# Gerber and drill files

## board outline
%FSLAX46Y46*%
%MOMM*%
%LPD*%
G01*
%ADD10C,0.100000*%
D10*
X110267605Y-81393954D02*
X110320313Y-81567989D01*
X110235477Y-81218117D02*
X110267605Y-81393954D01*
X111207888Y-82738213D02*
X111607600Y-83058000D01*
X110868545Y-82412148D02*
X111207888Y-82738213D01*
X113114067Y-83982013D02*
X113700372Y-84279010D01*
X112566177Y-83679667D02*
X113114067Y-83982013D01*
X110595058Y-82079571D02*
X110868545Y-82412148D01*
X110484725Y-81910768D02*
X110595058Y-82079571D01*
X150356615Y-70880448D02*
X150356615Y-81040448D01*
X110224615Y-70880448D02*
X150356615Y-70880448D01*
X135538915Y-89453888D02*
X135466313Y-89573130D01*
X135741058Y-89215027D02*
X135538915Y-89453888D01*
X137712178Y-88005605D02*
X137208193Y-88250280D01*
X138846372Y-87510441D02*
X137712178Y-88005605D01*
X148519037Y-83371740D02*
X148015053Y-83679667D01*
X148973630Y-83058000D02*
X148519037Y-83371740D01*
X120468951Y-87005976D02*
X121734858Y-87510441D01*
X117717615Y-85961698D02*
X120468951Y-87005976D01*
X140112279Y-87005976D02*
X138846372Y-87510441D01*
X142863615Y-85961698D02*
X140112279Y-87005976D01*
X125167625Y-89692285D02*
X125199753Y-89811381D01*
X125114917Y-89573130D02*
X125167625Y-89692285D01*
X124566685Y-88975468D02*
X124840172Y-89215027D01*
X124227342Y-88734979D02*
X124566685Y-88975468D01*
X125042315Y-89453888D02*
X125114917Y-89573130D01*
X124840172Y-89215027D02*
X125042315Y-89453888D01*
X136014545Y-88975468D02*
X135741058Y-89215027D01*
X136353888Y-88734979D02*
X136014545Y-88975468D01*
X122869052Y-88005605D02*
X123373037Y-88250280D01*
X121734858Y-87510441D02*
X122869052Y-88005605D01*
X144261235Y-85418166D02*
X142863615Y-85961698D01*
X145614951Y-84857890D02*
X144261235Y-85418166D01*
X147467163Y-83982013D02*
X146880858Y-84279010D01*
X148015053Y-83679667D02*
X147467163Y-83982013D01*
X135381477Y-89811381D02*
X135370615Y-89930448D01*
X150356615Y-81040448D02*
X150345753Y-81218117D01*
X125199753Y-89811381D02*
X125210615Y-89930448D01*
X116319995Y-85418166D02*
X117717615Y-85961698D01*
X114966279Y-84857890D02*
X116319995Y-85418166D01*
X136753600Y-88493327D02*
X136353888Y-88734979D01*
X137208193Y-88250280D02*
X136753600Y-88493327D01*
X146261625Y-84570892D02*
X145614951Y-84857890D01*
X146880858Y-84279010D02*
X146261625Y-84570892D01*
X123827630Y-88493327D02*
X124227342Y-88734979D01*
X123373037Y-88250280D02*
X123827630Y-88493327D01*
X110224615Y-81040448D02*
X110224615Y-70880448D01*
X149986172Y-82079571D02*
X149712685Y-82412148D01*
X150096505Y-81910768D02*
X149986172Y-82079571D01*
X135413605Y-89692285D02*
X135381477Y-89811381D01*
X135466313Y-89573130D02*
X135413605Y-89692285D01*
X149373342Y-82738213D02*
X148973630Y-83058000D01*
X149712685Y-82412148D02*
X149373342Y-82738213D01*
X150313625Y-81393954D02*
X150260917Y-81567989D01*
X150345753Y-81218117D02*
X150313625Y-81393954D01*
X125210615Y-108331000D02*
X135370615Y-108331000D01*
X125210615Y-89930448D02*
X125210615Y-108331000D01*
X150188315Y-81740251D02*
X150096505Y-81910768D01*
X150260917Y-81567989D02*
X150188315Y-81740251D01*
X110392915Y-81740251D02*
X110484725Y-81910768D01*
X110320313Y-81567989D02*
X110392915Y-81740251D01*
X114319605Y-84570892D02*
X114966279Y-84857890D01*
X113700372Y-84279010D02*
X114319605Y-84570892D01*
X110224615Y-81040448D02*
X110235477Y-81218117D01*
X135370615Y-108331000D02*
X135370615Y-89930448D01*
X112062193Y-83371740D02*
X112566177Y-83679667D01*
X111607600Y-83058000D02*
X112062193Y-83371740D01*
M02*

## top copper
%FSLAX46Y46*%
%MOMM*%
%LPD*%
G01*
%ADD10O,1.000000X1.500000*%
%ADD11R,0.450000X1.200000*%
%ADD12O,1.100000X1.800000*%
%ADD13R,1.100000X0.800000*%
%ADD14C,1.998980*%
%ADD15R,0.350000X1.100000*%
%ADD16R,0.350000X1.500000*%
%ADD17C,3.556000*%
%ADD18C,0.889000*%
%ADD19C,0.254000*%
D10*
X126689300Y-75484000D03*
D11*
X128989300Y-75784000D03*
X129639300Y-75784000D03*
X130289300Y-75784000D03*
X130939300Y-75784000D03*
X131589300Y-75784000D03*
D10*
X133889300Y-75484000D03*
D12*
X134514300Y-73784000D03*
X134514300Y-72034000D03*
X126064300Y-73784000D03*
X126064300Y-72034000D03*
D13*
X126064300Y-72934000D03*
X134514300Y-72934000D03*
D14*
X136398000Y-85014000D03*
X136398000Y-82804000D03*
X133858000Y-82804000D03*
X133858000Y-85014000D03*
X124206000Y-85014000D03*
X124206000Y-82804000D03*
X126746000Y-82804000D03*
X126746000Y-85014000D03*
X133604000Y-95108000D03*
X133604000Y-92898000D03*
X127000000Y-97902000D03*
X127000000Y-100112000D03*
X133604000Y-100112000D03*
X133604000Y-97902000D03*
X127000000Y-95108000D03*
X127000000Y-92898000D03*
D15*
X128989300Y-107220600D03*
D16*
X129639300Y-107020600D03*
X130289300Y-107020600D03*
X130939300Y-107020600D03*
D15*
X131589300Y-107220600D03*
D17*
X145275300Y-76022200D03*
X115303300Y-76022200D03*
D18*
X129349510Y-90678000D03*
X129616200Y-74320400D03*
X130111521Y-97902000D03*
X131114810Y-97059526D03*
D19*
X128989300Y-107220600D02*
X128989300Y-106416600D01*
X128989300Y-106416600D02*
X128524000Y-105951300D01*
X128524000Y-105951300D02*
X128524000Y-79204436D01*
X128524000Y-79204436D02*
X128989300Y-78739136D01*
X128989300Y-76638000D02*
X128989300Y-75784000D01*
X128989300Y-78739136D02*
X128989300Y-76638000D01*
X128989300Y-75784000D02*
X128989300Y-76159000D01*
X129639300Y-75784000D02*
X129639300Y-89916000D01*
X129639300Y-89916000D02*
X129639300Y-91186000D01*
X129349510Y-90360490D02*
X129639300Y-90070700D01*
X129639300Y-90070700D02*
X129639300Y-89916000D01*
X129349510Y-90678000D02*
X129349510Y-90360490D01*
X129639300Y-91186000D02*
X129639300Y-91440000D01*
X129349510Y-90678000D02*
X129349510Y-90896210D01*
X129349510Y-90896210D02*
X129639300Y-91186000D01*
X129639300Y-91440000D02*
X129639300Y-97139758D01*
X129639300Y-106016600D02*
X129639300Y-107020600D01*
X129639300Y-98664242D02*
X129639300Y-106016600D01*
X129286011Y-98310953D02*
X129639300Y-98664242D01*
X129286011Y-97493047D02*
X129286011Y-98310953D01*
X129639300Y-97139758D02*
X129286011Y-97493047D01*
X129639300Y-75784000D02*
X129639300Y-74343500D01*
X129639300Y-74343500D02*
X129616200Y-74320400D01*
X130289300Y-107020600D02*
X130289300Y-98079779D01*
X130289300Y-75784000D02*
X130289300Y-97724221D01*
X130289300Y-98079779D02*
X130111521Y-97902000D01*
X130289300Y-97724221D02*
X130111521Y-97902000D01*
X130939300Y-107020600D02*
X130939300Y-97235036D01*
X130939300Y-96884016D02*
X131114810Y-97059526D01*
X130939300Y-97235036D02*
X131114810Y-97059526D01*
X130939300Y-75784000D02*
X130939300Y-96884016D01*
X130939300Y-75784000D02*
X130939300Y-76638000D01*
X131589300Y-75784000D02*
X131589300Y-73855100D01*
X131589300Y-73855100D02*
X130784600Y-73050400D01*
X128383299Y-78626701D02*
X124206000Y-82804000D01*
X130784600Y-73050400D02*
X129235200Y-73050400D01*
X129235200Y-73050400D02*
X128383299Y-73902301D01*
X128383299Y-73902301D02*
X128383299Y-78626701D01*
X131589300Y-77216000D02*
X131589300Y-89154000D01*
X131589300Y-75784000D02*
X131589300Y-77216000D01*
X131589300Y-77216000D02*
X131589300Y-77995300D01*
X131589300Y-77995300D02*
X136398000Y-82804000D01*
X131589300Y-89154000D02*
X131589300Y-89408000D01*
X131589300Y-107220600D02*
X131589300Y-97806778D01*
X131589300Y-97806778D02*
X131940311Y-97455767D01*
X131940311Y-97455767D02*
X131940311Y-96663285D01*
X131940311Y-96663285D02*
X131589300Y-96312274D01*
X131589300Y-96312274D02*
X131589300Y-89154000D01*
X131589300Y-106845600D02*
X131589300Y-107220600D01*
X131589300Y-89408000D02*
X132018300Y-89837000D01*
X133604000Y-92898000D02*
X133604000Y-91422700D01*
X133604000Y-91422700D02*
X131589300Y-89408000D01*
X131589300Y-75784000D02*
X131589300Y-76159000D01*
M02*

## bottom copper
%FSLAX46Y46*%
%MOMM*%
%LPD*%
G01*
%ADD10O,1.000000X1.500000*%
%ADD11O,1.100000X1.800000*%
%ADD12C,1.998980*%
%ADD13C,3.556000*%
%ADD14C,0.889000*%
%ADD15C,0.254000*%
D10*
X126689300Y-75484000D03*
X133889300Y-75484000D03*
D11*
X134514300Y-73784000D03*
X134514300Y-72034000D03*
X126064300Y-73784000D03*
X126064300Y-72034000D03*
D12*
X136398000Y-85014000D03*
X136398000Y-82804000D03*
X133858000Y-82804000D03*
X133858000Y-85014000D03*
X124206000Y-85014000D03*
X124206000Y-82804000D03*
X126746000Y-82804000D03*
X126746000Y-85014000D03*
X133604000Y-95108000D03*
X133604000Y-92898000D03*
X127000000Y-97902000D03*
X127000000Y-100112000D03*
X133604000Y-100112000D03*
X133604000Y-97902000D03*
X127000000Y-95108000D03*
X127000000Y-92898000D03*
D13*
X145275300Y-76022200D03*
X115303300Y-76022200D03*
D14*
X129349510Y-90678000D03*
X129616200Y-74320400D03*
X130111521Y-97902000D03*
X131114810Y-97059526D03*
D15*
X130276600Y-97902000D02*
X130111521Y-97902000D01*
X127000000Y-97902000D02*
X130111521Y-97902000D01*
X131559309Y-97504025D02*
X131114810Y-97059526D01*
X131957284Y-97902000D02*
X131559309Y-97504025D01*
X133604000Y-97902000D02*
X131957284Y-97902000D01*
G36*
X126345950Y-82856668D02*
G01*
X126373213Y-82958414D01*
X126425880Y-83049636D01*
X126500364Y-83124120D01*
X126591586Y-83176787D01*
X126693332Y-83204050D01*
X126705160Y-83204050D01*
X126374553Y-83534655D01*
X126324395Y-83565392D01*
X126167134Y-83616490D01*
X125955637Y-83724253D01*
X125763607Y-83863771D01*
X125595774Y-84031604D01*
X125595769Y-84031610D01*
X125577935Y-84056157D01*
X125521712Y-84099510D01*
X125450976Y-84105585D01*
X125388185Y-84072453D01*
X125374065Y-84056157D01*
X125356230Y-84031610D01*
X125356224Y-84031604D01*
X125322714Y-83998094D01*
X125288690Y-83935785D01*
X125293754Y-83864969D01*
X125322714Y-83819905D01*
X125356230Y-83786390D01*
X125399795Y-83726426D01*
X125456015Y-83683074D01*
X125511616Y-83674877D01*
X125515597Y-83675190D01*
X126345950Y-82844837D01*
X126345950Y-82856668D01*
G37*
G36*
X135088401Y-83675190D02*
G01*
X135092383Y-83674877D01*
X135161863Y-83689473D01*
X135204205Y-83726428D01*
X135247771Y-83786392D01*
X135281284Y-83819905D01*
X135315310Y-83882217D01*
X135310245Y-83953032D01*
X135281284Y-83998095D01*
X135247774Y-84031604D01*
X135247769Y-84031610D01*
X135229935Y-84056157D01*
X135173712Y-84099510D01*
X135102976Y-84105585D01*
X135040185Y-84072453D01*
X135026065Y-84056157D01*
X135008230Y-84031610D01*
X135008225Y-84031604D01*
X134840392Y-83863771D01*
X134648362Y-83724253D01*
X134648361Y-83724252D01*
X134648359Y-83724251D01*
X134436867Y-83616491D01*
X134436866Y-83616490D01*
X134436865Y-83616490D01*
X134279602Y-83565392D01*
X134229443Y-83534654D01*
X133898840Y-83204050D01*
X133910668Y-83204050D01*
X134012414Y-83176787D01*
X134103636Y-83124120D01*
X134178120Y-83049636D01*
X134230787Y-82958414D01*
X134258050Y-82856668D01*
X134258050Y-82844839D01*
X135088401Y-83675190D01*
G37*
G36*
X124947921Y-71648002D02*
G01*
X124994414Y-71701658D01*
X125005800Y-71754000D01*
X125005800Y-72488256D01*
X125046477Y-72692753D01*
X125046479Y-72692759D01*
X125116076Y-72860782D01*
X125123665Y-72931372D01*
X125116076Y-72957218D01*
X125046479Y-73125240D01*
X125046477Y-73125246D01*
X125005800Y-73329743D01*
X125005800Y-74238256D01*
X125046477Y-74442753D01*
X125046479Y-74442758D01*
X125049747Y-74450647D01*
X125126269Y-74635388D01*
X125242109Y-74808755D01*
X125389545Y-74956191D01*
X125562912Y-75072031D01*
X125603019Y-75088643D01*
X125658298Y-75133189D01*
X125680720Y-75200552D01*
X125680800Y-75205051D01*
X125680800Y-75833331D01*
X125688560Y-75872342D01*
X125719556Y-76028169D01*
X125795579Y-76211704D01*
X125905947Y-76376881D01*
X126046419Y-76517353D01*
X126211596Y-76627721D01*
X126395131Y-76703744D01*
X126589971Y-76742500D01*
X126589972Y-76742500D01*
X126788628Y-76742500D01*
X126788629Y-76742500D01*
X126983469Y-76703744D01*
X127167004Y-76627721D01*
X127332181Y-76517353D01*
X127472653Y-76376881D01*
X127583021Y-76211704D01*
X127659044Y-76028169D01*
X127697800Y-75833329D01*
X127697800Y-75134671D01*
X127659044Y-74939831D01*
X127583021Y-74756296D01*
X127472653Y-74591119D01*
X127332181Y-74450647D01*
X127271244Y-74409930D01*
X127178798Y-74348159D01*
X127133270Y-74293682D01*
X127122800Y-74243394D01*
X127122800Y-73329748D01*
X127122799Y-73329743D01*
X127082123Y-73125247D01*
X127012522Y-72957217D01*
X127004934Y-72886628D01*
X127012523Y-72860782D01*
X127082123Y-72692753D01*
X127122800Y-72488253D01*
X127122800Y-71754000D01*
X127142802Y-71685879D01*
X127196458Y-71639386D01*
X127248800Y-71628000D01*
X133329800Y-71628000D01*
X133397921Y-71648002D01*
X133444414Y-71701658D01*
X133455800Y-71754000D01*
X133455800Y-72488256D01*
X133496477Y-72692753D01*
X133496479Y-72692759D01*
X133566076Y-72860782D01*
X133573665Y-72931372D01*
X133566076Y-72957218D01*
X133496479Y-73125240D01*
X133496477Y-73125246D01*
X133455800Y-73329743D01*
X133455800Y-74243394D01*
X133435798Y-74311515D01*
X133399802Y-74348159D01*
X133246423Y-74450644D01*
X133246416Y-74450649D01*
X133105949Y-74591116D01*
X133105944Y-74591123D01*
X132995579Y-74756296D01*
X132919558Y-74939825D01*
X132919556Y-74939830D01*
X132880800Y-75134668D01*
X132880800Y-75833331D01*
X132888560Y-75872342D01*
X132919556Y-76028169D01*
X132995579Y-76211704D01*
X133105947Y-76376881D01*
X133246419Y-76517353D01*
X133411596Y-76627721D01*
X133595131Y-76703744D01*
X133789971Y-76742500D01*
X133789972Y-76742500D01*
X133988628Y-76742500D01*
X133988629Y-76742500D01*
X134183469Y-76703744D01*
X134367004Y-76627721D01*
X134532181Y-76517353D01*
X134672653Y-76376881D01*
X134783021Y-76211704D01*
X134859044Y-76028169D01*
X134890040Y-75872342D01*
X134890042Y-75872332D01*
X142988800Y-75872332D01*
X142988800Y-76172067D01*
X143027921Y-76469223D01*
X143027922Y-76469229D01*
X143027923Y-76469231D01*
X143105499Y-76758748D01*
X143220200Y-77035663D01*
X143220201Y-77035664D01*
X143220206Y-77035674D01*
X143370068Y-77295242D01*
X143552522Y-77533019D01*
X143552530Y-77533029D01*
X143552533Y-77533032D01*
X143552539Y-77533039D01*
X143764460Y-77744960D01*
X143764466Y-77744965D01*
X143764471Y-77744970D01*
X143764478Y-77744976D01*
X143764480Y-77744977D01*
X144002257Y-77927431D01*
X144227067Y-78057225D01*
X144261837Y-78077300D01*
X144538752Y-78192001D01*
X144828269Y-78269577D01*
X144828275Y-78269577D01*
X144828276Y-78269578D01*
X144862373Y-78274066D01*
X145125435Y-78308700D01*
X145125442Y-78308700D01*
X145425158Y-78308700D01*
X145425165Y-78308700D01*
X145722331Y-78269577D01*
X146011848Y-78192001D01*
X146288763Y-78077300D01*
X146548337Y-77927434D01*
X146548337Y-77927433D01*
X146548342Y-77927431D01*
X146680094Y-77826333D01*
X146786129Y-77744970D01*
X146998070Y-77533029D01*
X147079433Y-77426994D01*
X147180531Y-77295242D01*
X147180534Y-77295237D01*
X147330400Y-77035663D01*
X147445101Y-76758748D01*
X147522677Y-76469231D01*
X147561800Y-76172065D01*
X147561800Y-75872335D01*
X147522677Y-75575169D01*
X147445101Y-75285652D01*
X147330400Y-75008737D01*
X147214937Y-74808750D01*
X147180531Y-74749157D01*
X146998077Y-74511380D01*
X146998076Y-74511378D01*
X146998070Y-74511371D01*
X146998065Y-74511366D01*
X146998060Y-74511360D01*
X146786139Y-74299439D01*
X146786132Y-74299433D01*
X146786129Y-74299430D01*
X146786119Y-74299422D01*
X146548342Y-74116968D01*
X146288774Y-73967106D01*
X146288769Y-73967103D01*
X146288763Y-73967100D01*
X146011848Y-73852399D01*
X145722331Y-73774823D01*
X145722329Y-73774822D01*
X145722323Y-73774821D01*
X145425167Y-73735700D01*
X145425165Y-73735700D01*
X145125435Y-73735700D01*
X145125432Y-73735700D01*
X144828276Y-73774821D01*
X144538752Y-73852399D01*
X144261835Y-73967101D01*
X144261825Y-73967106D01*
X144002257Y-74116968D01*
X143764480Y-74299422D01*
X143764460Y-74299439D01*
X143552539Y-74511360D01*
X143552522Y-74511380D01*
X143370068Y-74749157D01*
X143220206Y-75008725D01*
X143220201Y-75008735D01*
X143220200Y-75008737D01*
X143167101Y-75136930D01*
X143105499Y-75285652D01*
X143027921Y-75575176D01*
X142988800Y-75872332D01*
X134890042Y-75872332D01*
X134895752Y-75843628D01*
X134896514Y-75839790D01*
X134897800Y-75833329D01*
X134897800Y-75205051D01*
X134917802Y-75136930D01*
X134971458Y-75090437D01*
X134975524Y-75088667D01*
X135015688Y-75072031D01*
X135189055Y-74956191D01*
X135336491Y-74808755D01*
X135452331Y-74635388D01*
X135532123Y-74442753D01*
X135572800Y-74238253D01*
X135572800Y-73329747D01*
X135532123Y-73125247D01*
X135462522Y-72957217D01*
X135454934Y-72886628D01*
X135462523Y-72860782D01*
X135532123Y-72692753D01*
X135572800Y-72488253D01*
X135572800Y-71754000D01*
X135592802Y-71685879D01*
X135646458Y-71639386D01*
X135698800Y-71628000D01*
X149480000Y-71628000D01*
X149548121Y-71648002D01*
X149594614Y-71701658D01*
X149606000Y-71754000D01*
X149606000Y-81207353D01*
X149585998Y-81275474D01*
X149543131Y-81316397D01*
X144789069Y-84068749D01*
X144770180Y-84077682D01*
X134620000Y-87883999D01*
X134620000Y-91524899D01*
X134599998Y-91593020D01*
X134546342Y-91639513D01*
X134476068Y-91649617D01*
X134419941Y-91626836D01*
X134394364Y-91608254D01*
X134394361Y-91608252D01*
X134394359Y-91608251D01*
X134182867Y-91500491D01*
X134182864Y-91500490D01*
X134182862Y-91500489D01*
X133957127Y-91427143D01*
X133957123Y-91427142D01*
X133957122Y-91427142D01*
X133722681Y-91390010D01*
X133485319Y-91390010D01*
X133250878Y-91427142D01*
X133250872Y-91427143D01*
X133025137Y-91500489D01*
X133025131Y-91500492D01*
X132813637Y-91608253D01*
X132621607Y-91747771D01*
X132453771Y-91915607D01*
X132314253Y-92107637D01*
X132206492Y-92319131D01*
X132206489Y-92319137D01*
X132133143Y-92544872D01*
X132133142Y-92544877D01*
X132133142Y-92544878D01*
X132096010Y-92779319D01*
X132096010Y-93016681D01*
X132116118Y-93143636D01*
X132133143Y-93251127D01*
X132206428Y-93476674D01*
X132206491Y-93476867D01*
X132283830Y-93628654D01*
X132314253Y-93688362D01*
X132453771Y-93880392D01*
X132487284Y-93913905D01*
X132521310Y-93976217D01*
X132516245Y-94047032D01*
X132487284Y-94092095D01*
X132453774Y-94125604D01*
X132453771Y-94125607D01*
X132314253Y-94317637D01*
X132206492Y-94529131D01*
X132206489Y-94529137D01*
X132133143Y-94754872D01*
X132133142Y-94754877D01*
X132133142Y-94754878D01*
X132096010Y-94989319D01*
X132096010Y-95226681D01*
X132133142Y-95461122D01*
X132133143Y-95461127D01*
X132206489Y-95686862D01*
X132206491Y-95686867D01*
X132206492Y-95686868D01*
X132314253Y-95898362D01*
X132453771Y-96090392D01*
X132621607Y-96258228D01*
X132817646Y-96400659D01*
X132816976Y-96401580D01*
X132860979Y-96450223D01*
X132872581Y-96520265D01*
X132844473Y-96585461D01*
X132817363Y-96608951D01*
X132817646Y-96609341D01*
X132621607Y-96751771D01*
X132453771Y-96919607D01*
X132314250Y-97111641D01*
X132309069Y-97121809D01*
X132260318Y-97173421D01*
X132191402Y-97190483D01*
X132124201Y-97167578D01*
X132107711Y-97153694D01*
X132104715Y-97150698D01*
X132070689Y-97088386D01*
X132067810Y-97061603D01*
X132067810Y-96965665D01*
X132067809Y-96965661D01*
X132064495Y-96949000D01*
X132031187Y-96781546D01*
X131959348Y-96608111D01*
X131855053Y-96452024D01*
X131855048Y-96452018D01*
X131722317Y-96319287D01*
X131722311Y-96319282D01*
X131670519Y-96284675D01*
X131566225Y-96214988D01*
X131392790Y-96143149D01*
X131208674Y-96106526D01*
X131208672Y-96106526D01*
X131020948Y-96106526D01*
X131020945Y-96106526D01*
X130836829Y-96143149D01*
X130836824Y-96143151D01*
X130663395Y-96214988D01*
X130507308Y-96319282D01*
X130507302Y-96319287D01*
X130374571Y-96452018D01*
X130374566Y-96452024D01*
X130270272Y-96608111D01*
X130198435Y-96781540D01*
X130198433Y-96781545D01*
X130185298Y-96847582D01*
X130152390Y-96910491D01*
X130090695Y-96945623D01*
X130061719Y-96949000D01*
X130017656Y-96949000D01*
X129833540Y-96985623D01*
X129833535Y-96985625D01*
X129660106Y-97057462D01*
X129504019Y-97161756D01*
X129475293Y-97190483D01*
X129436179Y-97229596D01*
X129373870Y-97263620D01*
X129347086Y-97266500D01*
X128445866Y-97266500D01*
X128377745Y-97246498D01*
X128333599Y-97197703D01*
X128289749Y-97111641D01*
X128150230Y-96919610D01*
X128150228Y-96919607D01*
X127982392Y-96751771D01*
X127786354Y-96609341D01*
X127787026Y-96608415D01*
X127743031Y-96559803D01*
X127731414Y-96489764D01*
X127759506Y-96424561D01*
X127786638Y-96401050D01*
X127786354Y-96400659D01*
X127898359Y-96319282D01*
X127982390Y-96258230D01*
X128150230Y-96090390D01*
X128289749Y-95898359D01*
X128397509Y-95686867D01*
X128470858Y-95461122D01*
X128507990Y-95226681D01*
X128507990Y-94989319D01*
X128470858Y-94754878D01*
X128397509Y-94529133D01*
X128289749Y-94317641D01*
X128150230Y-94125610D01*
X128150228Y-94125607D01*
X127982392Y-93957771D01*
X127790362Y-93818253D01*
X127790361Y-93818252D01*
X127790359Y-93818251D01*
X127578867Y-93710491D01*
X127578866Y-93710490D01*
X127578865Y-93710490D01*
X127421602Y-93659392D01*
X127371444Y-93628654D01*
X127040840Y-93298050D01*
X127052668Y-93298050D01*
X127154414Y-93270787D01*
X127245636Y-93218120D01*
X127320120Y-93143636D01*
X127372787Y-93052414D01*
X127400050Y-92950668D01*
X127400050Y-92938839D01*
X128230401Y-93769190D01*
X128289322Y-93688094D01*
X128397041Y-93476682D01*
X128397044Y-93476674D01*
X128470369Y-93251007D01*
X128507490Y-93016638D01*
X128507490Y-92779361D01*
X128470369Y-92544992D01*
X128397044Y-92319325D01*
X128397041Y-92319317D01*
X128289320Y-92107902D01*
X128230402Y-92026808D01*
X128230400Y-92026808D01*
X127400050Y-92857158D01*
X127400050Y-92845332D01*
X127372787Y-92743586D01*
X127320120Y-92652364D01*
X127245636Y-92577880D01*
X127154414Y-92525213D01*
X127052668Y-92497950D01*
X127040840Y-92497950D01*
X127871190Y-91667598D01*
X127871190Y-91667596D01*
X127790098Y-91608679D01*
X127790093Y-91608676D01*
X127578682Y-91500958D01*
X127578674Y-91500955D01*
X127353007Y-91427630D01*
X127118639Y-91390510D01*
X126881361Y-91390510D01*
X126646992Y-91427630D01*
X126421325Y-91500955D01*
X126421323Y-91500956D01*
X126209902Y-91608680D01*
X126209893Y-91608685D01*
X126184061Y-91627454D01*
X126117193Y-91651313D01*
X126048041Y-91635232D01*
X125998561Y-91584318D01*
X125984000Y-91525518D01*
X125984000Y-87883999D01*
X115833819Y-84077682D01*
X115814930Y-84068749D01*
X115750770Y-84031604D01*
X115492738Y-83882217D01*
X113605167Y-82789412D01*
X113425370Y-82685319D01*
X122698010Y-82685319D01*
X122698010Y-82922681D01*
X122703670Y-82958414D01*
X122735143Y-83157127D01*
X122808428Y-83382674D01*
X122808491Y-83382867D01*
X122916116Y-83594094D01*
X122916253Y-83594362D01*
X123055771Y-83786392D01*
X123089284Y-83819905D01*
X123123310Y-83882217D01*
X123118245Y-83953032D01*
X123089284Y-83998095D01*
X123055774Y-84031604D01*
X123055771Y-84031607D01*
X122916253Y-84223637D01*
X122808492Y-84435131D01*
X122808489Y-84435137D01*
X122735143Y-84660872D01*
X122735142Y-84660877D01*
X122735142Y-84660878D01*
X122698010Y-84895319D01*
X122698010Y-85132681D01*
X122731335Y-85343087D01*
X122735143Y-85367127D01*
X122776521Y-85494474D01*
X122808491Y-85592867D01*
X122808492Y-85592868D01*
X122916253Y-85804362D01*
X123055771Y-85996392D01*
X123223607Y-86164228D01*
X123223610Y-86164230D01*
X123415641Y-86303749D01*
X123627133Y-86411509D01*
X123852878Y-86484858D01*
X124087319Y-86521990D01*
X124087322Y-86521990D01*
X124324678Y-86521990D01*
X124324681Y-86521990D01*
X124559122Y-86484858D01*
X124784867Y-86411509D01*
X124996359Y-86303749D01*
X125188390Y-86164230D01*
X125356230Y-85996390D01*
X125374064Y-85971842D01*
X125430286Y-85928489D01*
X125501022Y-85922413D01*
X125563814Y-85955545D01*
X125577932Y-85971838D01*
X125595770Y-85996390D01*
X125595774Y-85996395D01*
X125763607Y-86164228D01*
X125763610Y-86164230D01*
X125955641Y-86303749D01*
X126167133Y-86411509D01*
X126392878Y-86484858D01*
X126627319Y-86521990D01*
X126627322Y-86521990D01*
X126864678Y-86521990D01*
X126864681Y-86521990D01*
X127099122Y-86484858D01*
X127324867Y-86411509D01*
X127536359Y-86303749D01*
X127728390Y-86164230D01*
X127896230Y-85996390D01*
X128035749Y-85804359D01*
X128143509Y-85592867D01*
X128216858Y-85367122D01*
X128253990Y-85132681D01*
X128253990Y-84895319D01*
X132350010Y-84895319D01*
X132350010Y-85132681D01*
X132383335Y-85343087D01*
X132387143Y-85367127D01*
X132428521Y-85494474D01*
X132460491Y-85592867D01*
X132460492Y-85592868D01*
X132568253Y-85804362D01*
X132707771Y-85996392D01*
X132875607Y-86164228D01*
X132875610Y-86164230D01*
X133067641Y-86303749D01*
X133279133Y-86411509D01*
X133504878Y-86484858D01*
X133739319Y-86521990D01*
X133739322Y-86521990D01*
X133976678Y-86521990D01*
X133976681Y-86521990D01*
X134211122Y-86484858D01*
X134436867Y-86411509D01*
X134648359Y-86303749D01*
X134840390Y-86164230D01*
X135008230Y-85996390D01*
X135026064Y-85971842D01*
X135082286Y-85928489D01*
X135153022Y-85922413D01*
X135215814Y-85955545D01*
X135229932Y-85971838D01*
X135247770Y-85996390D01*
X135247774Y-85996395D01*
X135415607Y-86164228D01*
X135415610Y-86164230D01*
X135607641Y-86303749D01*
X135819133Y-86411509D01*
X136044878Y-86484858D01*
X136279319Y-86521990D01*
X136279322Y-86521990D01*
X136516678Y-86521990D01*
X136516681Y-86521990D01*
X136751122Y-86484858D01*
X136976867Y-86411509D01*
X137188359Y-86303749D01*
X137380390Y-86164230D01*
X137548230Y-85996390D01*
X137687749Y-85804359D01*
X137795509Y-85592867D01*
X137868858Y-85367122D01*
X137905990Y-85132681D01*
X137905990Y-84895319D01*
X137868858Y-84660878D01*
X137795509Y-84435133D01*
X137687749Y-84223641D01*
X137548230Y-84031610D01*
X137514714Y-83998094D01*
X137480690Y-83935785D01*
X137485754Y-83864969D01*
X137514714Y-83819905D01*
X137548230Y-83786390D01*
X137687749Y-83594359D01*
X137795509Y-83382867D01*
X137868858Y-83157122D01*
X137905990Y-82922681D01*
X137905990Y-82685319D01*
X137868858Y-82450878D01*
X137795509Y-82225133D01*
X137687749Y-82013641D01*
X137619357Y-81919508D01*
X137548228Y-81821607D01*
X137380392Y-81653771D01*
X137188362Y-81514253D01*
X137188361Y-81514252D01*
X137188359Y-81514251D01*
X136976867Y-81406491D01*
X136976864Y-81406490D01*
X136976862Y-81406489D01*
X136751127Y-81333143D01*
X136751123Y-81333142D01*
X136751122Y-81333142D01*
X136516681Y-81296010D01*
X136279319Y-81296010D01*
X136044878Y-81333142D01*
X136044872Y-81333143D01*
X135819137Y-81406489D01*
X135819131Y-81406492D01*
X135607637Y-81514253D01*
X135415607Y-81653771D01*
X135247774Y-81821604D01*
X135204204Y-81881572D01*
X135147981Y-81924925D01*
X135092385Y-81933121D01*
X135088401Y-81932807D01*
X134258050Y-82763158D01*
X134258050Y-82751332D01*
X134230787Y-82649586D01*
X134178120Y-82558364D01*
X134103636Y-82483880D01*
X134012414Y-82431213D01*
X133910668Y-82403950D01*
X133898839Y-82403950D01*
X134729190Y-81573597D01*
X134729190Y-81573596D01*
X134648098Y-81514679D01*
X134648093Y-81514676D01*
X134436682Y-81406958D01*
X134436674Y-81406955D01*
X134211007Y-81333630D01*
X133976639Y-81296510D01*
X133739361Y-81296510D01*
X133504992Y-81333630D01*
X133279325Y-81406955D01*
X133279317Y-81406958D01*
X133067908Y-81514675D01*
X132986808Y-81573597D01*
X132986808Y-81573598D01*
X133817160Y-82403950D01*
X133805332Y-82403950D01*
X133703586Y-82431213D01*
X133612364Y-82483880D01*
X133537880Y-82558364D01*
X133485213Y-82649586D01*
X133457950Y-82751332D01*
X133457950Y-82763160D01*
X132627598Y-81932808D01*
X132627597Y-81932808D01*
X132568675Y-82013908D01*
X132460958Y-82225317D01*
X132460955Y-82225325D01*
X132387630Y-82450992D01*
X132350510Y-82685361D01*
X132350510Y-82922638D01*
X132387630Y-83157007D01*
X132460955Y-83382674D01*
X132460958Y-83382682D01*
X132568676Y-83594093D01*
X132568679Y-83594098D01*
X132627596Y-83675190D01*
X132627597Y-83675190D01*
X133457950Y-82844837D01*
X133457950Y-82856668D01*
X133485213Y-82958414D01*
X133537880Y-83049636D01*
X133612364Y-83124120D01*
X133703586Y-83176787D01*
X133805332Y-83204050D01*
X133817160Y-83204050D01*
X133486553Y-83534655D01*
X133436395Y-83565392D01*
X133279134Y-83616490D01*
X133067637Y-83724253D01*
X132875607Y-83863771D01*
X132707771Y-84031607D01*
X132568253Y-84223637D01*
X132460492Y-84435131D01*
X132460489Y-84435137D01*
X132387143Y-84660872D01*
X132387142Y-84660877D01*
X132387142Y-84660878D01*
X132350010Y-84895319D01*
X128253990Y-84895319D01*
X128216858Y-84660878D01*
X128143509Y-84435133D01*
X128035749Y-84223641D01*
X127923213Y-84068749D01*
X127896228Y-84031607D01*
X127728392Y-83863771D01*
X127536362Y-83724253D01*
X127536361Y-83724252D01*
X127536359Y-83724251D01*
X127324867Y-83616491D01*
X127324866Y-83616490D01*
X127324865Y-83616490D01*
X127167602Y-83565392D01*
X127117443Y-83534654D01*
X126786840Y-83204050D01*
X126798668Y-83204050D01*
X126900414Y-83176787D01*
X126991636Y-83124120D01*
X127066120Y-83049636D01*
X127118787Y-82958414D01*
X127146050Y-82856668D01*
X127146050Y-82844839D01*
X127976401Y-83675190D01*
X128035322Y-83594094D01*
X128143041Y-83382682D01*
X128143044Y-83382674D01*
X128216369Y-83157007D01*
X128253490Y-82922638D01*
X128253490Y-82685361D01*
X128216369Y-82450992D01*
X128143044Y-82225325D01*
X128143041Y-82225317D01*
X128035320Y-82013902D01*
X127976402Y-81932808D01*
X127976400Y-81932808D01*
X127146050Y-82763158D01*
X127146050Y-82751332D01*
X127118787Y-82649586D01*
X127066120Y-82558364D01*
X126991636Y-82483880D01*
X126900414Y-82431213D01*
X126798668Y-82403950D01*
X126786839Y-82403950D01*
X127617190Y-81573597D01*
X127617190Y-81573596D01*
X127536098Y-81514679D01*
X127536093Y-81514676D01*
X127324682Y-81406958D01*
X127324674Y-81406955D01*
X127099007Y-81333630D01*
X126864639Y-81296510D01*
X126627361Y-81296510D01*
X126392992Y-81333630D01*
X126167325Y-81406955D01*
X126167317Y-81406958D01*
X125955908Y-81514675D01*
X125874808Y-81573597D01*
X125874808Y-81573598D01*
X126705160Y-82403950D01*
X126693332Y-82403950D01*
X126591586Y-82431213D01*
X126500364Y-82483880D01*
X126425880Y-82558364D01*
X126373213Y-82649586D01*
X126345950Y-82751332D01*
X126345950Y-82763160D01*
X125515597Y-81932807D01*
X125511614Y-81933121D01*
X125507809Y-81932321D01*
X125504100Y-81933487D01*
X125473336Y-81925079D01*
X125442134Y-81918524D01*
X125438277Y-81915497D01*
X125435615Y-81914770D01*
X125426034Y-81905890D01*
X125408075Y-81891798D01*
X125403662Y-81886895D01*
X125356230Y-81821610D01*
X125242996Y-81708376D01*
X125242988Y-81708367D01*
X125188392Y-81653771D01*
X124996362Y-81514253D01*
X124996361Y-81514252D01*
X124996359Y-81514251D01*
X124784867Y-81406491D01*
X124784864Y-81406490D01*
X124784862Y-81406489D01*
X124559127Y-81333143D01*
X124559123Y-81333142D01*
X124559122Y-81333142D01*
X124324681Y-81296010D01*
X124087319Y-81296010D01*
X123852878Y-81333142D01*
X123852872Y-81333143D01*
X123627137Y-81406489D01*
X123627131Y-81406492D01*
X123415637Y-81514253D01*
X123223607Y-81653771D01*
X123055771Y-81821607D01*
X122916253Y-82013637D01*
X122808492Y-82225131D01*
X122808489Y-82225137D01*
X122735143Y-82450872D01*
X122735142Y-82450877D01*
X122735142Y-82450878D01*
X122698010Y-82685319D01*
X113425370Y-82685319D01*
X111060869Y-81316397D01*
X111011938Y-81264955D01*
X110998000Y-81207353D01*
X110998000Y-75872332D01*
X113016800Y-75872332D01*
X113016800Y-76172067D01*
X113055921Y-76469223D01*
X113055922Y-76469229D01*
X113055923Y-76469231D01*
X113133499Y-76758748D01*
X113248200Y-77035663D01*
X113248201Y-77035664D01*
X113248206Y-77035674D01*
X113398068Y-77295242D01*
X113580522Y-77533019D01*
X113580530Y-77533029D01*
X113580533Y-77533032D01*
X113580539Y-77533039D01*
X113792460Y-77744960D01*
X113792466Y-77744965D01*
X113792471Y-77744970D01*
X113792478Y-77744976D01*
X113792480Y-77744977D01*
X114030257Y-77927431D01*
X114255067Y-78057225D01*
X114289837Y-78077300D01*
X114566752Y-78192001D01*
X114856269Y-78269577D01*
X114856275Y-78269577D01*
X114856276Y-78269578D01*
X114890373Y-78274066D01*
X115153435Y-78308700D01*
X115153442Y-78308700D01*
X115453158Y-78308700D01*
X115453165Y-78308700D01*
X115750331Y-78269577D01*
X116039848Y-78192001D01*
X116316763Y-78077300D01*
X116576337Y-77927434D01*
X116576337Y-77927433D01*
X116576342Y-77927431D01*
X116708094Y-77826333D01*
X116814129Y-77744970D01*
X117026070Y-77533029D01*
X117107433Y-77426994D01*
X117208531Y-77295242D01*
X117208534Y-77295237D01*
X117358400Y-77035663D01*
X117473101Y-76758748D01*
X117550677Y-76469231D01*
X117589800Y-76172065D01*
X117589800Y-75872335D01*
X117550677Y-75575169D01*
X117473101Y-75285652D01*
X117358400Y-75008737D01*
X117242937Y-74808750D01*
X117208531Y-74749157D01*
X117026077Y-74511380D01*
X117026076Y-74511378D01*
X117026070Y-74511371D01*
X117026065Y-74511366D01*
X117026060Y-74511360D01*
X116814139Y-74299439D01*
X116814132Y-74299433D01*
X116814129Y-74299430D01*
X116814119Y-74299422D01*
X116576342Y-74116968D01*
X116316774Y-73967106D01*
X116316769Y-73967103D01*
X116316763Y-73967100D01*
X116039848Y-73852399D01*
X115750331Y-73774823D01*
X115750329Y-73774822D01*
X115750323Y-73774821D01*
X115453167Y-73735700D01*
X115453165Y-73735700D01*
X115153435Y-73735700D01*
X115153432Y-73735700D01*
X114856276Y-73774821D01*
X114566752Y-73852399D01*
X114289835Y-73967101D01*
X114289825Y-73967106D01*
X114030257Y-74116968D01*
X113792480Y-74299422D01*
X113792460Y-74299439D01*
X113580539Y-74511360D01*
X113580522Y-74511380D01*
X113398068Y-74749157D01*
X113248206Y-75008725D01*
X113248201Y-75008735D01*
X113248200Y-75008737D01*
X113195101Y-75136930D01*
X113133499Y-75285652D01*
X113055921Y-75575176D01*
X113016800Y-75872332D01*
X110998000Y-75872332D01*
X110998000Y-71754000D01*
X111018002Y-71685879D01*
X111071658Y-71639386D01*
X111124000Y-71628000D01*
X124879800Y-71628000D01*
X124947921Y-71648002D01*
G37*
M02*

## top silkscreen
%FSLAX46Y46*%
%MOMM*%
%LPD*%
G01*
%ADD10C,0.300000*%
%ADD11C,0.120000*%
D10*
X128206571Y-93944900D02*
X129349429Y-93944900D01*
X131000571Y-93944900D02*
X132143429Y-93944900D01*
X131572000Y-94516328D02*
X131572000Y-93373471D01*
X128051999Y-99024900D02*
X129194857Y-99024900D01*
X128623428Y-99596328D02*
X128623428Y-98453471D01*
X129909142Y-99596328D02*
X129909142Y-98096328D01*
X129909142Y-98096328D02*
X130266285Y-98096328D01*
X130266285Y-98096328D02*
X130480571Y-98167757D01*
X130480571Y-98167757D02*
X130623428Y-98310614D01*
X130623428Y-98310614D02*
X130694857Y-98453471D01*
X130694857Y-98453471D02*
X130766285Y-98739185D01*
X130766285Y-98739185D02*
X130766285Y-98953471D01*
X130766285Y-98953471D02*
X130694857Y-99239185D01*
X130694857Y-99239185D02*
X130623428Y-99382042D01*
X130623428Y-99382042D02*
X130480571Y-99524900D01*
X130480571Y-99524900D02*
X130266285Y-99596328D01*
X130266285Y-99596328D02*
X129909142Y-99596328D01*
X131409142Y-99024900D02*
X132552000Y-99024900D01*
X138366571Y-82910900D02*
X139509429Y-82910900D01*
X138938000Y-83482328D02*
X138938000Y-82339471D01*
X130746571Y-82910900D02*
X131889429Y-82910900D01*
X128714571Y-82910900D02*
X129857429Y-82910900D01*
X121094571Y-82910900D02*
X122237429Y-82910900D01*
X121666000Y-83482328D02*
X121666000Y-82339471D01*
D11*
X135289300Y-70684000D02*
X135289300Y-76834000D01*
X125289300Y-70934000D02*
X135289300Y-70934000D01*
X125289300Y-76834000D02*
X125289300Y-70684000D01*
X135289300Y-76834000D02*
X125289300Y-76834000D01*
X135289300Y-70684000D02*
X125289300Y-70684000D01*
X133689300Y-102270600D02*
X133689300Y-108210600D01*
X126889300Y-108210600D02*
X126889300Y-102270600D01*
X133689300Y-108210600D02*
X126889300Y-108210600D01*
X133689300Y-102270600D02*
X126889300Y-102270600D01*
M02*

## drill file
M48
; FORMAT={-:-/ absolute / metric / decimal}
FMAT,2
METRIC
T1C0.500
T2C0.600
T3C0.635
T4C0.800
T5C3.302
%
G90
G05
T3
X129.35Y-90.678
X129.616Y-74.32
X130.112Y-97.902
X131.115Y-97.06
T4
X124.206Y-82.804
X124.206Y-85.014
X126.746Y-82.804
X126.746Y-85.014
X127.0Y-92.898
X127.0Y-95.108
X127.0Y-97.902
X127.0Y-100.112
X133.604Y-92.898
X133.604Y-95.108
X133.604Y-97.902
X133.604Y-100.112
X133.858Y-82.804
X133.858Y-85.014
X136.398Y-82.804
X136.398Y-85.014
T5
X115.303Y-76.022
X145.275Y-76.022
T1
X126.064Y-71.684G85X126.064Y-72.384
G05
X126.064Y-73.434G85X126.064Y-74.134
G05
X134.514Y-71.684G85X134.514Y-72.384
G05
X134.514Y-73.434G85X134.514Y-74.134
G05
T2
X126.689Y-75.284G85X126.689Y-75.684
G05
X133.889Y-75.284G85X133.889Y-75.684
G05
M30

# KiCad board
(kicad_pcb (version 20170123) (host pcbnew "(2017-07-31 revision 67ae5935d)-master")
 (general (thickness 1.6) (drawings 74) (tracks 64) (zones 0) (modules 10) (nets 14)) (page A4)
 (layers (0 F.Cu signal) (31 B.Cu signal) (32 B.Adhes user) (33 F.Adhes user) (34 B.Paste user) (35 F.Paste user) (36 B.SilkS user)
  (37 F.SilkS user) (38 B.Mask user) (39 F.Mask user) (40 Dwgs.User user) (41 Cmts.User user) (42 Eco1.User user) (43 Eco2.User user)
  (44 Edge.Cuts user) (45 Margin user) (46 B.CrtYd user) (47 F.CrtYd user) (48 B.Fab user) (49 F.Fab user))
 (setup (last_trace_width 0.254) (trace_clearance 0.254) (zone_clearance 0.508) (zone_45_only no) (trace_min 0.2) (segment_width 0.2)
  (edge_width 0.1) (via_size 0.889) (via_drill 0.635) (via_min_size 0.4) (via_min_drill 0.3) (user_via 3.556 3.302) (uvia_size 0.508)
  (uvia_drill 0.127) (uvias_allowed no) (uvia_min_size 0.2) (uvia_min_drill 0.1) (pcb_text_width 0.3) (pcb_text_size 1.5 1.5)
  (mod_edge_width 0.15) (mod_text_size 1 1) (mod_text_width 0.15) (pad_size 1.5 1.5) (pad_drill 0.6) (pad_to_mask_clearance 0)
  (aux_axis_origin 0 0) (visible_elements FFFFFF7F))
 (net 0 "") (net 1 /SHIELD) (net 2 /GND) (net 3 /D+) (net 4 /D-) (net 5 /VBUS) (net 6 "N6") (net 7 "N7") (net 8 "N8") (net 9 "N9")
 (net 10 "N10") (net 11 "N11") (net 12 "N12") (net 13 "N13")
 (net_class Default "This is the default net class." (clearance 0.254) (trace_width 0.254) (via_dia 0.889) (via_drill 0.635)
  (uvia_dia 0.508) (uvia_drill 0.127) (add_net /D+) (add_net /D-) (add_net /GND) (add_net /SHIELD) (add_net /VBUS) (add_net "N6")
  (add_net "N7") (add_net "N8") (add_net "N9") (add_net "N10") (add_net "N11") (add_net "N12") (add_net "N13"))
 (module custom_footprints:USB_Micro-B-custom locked (layer F.Cu) (at 130.2893 75.184 180)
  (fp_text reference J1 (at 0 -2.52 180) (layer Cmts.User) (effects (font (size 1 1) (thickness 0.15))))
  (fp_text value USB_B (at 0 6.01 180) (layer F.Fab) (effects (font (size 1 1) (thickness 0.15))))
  (fp_line (start -5 4.5) (end -5 -1.65) (layer F.SilkS) (width 0.12))
  (fp_line (start 5 4.25) (end -5 4.25) (layer F.SilkS) (width 0.12))
  (fp_line (start 5 -1.65) (end 5 4.5) (layer F.SilkS) (width 0.12))
  (fp_line (start -5 -1.65) (end 5 -1.65) (layer F.SilkS) (width 0.12))
  (fp_line (start -5 4.5) (end 5 4.5) (layer F.SilkS) (width 0.12))
  (pad "" thru_hole oval (at 3.6 -0.3 270) (size 1.5 1) (drill oval 1 0.6) (layers *.Cu *.Mask))
  (pad 5 smd rect (at 1.3 -0.6 270) (size 1.2 0.45) (layers F.Cu F.Paste F.Mask) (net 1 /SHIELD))
  (pad 4 smd rect (at 0.65 -0.6 270) (size 1.2 0.45) (layers F.Cu F.Paste F.Mask) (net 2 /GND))
  (pad 3 smd rect (at 0 -0.6 270) (size 1.2 0.45) (layers F.Cu F.Paste F.Mask) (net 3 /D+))
  (pad 2 smd rect (at -0.65 -0.6 270) (size 1.2 0.45) (layers F.Cu F.Paste F.Mask) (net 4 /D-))
  (pad 1 smd rect (at -1.3 -0.6 270) (size 1.2 0.45) (layers F.Cu F.Paste F.Mask) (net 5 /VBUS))
  (pad "" thru_hole oval (at -3.6 -0.3 270) (size 1.5 1) (drill oval 1 0.6) (layers *.Cu *.Mask))
  (pad "" thru_hole oval (at -4.225 1.4 270) (size 1.8 1.1) (drill oval 1.2 0.5) (layers *.Cu *.Mask))
  (pad "" thru_hole oval (at -4.225 3.15 270) (size 1.8 1.1) (drill oval 1.2 0.5) (layers *.Cu *.Mask))
  (pad "" thru_hole oval (at 4.225 1.4 270) (size 1.8 1.1) (drill oval 1.2 0.5) (layers *.Cu *.Mask))
  (pad "" thru_hole oval (at 4.225 3.15 270) (size 1.8 1.1) (drill oval 1.2 0.5) (layers *.Cu *.Mask))
  (pad "" smd rect (at 4.225 2.25 270) (size 0.8 1.1) (layers F.Cu F.Paste F.Mask))
  (pad "" smd rect (at -4.225 2.25 270) (size 0.8 1.1) (layers F.Cu F.Paste F.Mask)))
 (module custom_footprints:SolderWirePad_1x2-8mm (layer F.Cu) (at 136.398 83.914 270)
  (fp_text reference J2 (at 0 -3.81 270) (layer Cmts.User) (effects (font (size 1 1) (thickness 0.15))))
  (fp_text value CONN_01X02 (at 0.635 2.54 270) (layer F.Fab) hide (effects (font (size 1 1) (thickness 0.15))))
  (pad 2 thru_hole circle (at 1.1 0 270) (size 1.99898 1.99898) (drill 0.8001) (layers *.Cu *.Mask) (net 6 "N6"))
  (pad 1 thru_hole circle (at -1.11 0 270) (size 1.99898 1.99898) (drill 0.8001) (layers *.Cu *.Mask) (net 5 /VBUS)))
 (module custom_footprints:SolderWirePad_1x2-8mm (layer F.Cu) (at 133.858 83.914 270)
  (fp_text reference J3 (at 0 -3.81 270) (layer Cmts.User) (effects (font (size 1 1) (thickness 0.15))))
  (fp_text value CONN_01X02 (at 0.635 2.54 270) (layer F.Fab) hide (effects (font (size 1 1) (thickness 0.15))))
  (pad 1 thru_hole circle (at -1.11 0 270) (size 1.99898 1.99898) (drill 0.8001) (layers *.Cu *.Mask) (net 2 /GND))
  (pad 2 thru_hole circle (at 1.1 0 270) (size 1.99898 1.99898) (drill 0.8001) (layers *.Cu *.Mask) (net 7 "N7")))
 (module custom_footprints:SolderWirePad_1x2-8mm (layer F.Cu) (at 124.206 83.914 270)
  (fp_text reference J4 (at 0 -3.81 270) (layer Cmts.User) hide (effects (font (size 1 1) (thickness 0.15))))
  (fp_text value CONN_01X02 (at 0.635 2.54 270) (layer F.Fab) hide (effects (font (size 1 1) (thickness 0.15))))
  (pad 2 thru_hole circle (at 1.1 0 270) (size 1.99898 1.99898) (drill 0.8001) (layers *.Cu *.Mask) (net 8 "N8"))
  (pad 1 thru_hole circle (at -1.11 0 270) (size 1.99898 1.99898) (drill 0.8001) (layers *.Cu *.Mask) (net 5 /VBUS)))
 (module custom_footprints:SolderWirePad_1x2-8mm (layer F.Cu) (at 126.746 83.914 270)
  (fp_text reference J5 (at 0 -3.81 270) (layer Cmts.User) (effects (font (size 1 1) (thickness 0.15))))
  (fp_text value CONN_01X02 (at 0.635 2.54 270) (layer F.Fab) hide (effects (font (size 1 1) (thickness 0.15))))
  (pad 1 thru_hole circle (at -1.11 0 270) (size 1.99898 1.99898) (drill 0.8001) (layers *.Cu *.Mask) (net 2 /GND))
  (pad 2 thru_hole circle (at 1.1 0 270) (size 1.99898 1.99898) (drill 0.8001) (layers *.Cu *.Mask) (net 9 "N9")))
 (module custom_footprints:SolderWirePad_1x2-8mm (layer F.Cu) (at 133.604 94.008 270)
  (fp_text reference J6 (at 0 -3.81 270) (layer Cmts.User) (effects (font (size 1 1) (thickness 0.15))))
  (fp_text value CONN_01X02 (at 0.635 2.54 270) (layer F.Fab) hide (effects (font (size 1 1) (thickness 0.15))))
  (pad 2 thru_hole circle (at 1.1 0 270) (size 1.99898 1.99898) (drill 0.8001) (layers *.Cu *.Mask) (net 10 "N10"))
  (pad 1 thru_hole circle (at -1.11 0 270) (size 1.99898 1.99898) (drill 0.8001) (layers *.Cu *.Mask) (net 5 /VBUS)))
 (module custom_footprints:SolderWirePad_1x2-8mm (layer F.Cu) (at 127 99.012 270)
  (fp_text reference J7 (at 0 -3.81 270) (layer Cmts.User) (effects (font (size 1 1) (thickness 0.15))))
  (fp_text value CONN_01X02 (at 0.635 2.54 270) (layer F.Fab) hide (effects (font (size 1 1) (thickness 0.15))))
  (pad 1 thru_hole circle (at -1.11 0 270) (size 1.99898 1.99898) (drill 0.8001) (layers *.Cu *.Mask) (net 3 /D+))
  (pad 2 thru_hole circle (at 1.1 0 270) (size 1.99898 1.99898) (drill 0.8001) (layers *.Cu *.Mask) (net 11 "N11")))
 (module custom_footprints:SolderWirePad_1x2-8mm (layer F.Cu) (at 133.604 99.012 270)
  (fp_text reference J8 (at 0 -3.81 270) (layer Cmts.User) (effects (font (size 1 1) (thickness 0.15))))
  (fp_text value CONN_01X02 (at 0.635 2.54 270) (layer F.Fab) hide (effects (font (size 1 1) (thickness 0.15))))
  (pad 2 thru_hole circle (at 1.1 0 270) (size 1.99898 1.99898) (drill 0.8001) (layers *.Cu *.Mask) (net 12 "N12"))
  (pad 1 thru_hole circle (at -1.11 0 270) (size 1.99898 1.99898) (drill 0.8001) (layers *.Cu *.Mask) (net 4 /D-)))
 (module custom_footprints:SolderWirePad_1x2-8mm (layer F.Cu) (at 127 94.008 270)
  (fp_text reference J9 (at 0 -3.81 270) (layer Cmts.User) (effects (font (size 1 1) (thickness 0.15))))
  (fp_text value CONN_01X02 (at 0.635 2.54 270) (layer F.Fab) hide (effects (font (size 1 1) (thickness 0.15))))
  (pad 2 thru_hole circle (at 1.1 0 270) (size 1.99898 1.99898) (drill 0.8001) (layers *.Cu *.Mask) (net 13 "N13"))
  (pad 1 thru_hole circle (at -1.11 0 270) (size 1.99898 1.99898) (drill 0.8001) (layers *.Cu *.Mask) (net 2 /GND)))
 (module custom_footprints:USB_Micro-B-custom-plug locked (layer F.Cu) (at 130.2893 107.0206 180)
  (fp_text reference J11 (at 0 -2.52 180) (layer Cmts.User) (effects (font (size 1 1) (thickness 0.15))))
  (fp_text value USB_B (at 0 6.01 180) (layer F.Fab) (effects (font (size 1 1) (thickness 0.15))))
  (fp_line (start -3.4 4.75) (end -3.4 -1.19) (layer F.SilkS) (width 0.12))
  (fp_line (start 3.4 -1.19) (end 3.4 4.75) (layer F.SilkS) (width 0.12))
  (fp_line (start -3.4 -1.19) (end 3.4 -1.19) (layer F.SilkS) (width 0.12))
  (fp_line (start -3.4 4.75) (end 3.4 4.75) (layer F.SilkS) (width 0.12))
  (pad 5 smd rect (at 1.3 -0.2 270) (size 1.1 0.35) (layers F.Cu F.Paste F.Mask) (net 1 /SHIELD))
  (pad 4 smd rect (at 0.65 0 270) (size 1.5 0.35) (layers F.Cu F.Paste F.Mask) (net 2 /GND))
  (pad 3 smd rect (at 0 0 270) (size 1.5 0.35) (layers F.Cu F.Paste F.Mask) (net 3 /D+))
  (pad 2 smd rect (at -0.65 0 270) (size 1.5 0.35) (layers F.Cu F.Paste F.Mask) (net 4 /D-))
  (pad 1 smd rect (at -1.3 -0.2 270) (size 1.1 0.35) (layers F.Cu F.Paste F.Mask) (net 5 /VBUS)))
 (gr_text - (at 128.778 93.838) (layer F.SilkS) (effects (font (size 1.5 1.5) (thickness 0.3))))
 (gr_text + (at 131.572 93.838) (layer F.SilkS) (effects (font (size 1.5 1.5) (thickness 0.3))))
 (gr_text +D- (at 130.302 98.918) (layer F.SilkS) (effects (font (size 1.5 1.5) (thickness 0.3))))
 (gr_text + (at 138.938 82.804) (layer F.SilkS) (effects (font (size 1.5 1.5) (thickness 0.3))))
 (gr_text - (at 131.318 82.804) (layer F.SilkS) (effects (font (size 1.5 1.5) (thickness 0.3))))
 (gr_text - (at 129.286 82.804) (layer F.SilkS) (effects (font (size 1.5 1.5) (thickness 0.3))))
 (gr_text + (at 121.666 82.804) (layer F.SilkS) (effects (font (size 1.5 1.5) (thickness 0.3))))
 (gr_line (start 110.267605 81.393954) (end 110.320313 81.567989) (layer Edge.Cuts) (width 0.1))
 (gr_line (start 110.235477 81.218117) (end 110.267605 81.393954) (layer Edge.Cuts) (width 0.1))
 (gr_line (start 111.207888 82.738213) (end 111.6076 83.058) (layer Edge.Cuts) (width 0.1))
 (gr_line (start 110.868545 82.412148) (end 111.207888 82.738213) (layer Edge.Cuts) (width 0.1))
 (gr_line (start 113.114067 83.982013) (end 113.700372 84.27901) (layer Edge.Cuts) (width 0.1))
 (gr_line (start 112.566177 83.679667) (end 113.114067 83.982013) (layer Edge.Cuts) (width 0.1))
 (gr_line (start 110.595058 82.079571) (end 110.868545 82.412148) (layer Edge.Cuts) (width 0.1))
 (gr_line (start 110.484725 81.910768) (end 110.595058 82.079571) (layer Edge.Cuts) (width 0.1))
 (gr_line (start 150.356615 70.880448) (end 150.356615 81.040448) (layer Edge.Cuts) (width 0.1))
 (gr_line (start 110.224615 70.880448) (end 150.356615 70.880448) (layer Edge.Cuts) (width 0.1))
 (gr_line (start 135.538915 89.453888) (end 135.466313 89.57313) (layer Edge.Cuts) (width 0.1))
 (gr_line (start 135.741058 89.215027) (end 135.538915 89.453888) (layer Edge.Cuts) (width 0.1))
 (gr_line (start 137.712178 88.005605) (end 137.208193 88.25028) (layer Edge.Cuts) (width 0.1))
 (gr_line (start 138.846372 87.510441) (end 137.712178 88.005605) (layer Edge.Cuts) (width 0.1))
 (gr_line (start 148.519037 83.37174) (end 148.015053 83.679667) (layer Edge.Cuts) (width 0.1))
 (gr_line (start 148.97363 83.058) (end 148.519037 83.37174) (layer Edge.Cuts) (width 0.1))
 (gr_line (start 120.468951 87.005976) (end 121.734858 87.510441) (layer Edge.Cuts) (width 0.1))
 (gr_line (start 117.717615 85.961698) (end 120.468951 87.005976) (layer Edge.Cuts) (width 0.1))
 (gr_line (start 140.112279 87.005976) (end 138.846372 87.510441) (layer Edge.Cuts) (width 0.1))
 (gr_line (start 142.863615 85.961698) (end 140.112279 87.005976) (layer Edge.Cuts) (width 0.1))
 (gr_line (start 125.167625 89.692285) (end 125.199753 89.811381) (layer Edge.Cuts) (width 0.1))
 (gr_line (start 125.114917 89.57313) (end 125.167625 89.692285) (layer Edge.Cuts) (width 0.1))
 (gr_line (start 124.566685 88.975468) (end 124.840172 89.215027) (layer Edge.Cuts) (width 0.1))
 (gr_line (start 124.227342 88.734979) (end 124.566685 88.975468) (layer Edge.Cuts) (width 0.1))
 (gr_line (start 125.042315 89.453888) (end 125.114917 89.57313) (layer Edge.Cuts) (width 0.1))
 (gr_line (start 124.840172 89.215027) (end 125.042315 89.453888) (layer Edge.Cuts) (width 0.1))
 (gr_line (start 136.014545 88.975468) (end 135.741058 89.215027) (layer Edge.Cuts) (width 0.1))
 (gr_line (start 136.353888 88.734979) (end 136.014545 88.975468) (layer Edge.Cuts) (width 0.1))
 (gr_line (start 122.869052 88.005605) (end 123.373037 88.25028) (layer Edge.Cuts) (width 0.1))
 (gr_line (start 121.734858 87.510441) (end 122.869052 88.005605) (layer Edge.Cuts) (width 0.1))
 (gr_line (start 144.261235 85.418166) (end 142.863615 85.961698) (layer Edge.Cuts) (width 0.1))
 (gr_line (start 145.614951 84.85789) (end 144.261235 85.418166) (layer Edge.Cuts) (width 0.1))
 (gr_line (start 147.467163 83.982013) (end 146.880858 84.27901) (layer Edge.Cuts) (width 0.1))
 (gr_line (start 148.015053 83.679667) (end 147.467163 83.982013) (layer Edge.Cuts) (width 0.1))
 (gr_line (start 135.381477 89.811381) (end 135.370615 89.930448) (layer Edge.Cuts) (width 0.1))
 (gr_line (start 150.356615 81.040448) (end 150.345753 81.218117) (layer Edge.Cuts) (width 0.1))
 (gr_line (start 125.199753 89.811381) (end 125.210615 89.930448) (layer Edge.Cuts) (width 0.1))
 (gr_line (start 116.319995 85.418166) (end 117.717615 85.961698) (layer Edge.Cuts) (width 0.1))
 (gr_line (start 114.966279 84.85789) (end 116.319995 85.418166) (layer Edge.Cuts) (width 0.1))
 (gr_line (start 136.7536 88.493327) (end 136.353888 88.734979) (layer Edge.Cuts) (width 0.1))
 (gr_line (start 137.208193 88.25028) (end 136.7536 88.493327) (layer Edge.Cuts) (width 0.1))
 (gr_line (start 146.261625 84.570892) (end 145.614951 84.85789) (layer Edge.Cuts) (width 0.1))
 (gr_line (start 146.880858 84.27901) (end 146.261625 84.570892) (layer Edge.Cuts) (width 0.1))
 (gr_line (start 123.82763 88.493327) (end 124.227342 88.734979) (layer Edge.Cuts) (width 0.1))
 (gr_line (start 123.373037 88.25028) (end 123.82763 88.493327) (layer Edge.Cuts) (width 0.1))
 (gr_line (start 110.224615 81.040448) (end 110.224615 70.880448) (layer Edge.Cuts) (width 0.1))
 (gr_line (start 149.986172 82.079571) (end 149.712685 82.412148) (layer Edge.Cuts) (width 0.1))
 (gr_line (start 150.096505 81.910768) (end 149.986172 82.079571) (layer Edge.Cuts) (width 0.1))
 (gr_line (start 135.413605 89.692285) (end 135.381477 89.811381) (layer Edge.Cuts) (width 0.1))
 (gr_line (start 135.466313 89.57313) (end 135.413605 89.692285) (layer Edge.Cuts) (width 0.1))
 (gr_line (start 149.373342 82.738213) (end 148.97363 83.058) (layer Edge.Cuts) (width 0.1))
 (gr_line (start 149.712685 82.412148) (end 149.373342 82.738213) (layer Edge.Cuts) (width 0.1))
 (gr_line (start 150.313625 81.393954) (end 150.260917 81.567989) (layer Edge.Cuts) (width 0.1))
 (gr_line (start 150.345753 81.218117) (end 150.313625 81.393954) (layer Edge.Cuts) (width 0.1))
 (gr_line (start 125.210615 108.331) (end 135.370615 108.331) (layer Edge.Cuts) (width 0.1))
 (gr_line (start 125.210615 89.930448) (end 125.210615 108.331) (layer Edge.Cuts) (width 0.1))
 (gr_line (start 150.188315 81.740251) (end 150.096505 81.910768) (layer Edge.Cuts) (width 0.1))
 (gr_line (start 150.260917 81.567989) (end 150.188315 81.740251) (layer Edge.Cuts) (width 0.1))
 (gr_line (start 110.392915 81.740251) (end 110.484725 81.910768) (layer Edge.Cuts) (width 0.1))
 (gr_line (start 110.320313 81.567989) (end 110.392915 81.740251) (layer Edge.Cuts) (width 0.1))
 (gr_line (start 114.319605 84.570892) (end 114.966279 84.85789) (layer Edge.Cuts) (width 0.1))
 (gr_line (start 113.700372 84.27901) (end 114.319605 84.570892) (layer Edge.Cuts) (width 0.1))
 (gr_line (start 110.224615 81.040448) (end 110.235477 81.218117) (layer Edge.Cuts) (width 0.1))
 (gr_line (start 135.370615 108.331) (end 135.370615 89.930448) (layer Edge.Cuts) (width 0.1))
 (gr_line (start 112.062193 83.37174) (end 112.566177 83.679667) (layer Edge.Cuts) (width 0.1))
 (gr_line (start 111.6076 83.058) (end 112.062193 83.37174) (layer Edge.Cuts) (width 0.1))
 (via (at 145.2753 76.0222) (size 3.556) (drill 3.302) (layers F.Cu B.Cu) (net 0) (status 40000))
 (via (at 115.3033 76.0222) (size 3.556) (drill 3.302) (layers F.Cu B.Cu) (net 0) (status 40000))
 (segment (start 128.9893 107.2206) (end 128.9893 106.4166) (width 0.254) (layer F.Cu) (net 1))
 (segment (start 128.9893 106.4166) (end 128.524 105.9513) (width 0.254) (layer F.Cu) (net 1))
 (segment (start 128.524 105.9513) (end 128.524 79.204436) (width 0.254) (layer F.Cu) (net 1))
 (segment (start 128.524 79.204436) (end 128.9893 78.739136) (width 0.254) (layer F.Cu) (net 1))
 (segment (start 128.9893 76.638) (end 128.9893 75.784) (width 0.254) (layer F.Cu) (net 1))
 (segment (start 128.9893 78.739136) (end 128.9893 76.638) (width 0.254) (layer F.Cu) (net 1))
 (segment (start 128.9893 75.784) (end 128.9893 76.159) (width 0.254) (layer F.Cu) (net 1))
 (segment (start 129.6393 75.784) (end 129.6393 89.916) (width 0.254) (layer F.Cu) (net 2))
 (segment (start 129.6393 89.916) (end 129.6393 91.186) (width 0.254) (layer F.Cu) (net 2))
 (segment (start 129.34951 90.36049) (end 129.6393 90.0707) (width 0.254) (layer F.Cu) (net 2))
 (segment (start 129.6393 90.0707) (end 129.6393 89.916) (width 0.254) (layer F.Cu) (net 2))
 (segment (start 129.34951 90.678) (end 129.34951 90.36049) (width 0.254) (layer F.Cu) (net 2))
 (segment (start 129.6393 91.186) (end 129.6393 91.44) (width 0.254) (layer F.Cu) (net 2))
 (segment (start 129.34951 90.678) (end 129.34951 90.89621) (width 0.254) (layer F.Cu) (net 2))
 (segment (start 129.34951 90.89621) (end 129.6393 91.186) (width 0.254) (layer F.Cu) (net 2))
 (via (at 129.34951 90.678) (size 0.889) (drill 0.635) (layers F.Cu B.Cu) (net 2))
 (segment (start 129.6393 91.44) (end 129.6393 97.139758) (width 0.254) (layer F.Cu) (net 2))
 (segment (start 129.6393 106.0166) (end 129.6393 107.0206) (width 0.254) (layer F.Cu) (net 2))
 (segment (start 129.6393 98.664242) (end 129.6393 106.0166) (width 0.254) (layer F.Cu) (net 2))
 (segment (start 129.286011 98.310953) (end 129.6393 98.664242) (width 0.254) (layer F.Cu) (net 2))
 (segment (start 129.286011 97.493047) (end 129.286011 98.310953) (width 0.254) (layer F.Cu) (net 2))
 (segment (start 129.6393 97.139758) (end 129.286011 97.493047) (width 0.254) (layer F.Cu) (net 2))
 (segment (start 129.6393 75.784) (end 129.6393 74.3435) (width 0.254) (layer F.Cu) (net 2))
 (segment (start 129.6393 74.3435) (end 129.6162 74.3204) (width 0.254) (layer F.Cu) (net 2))
 (via (at 129.6162 74.3204) (size 0.889) (drill 0.635) (layers F.Cu B.Cu) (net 2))
 (segment (start 130.2893 107.0206) (end 130.2893 98.079779) (width 0.254) (layer F.Cu) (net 3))
 (segment (start 130.2893 75.784) (end 130.2893 97.724221) (width 0.254) (layer F.Cu) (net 3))
 (segment (start 130.2893 98.079779) (end 130.111521 97.902) (width 0.254) (layer F.Cu) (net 3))
 (via (at 130.111521 97.902) (size 0.889) (drill 0.635) (layers F.Cu B.Cu) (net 3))
 (segment (start 130.2766 97.902) (end 130.111521 97.902) (width 0.254) (layer B.Cu) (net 3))
 (segment (start 127 97.902) (end 130.111521 97.902) (width 0.254) (layer B.Cu) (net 3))
 (segment (start 130.2893 97.724221) (end 130.111521 97.902) (width 0.254) (layer F.Cu) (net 3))
 (segment (start 131.559309 97.504025) (end 131.11481 97.059526) (width 0.254) (layer B.Cu) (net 4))
 (segment (start 131.957284 97.902) (end 131.559309 97.504025) (width 0.254) (layer B.Cu) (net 4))
 (segment (start 133.604 97.902) (end 131.957284 97.902) (width 0.254) (layer B.Cu) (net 4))
 (segment (start 130.9393 107.0206) (end 130.9393 97.235036) (width 0.254) (layer F.Cu) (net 4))
 (segment (start 130.9393 96.884016) (end 131.11481 97.059526) (width 0.254) (layer F.Cu) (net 4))
 (segment (start 130.9393 97.235036) (end 131.11481 97.059526) (width 0.254) (layer F.Cu) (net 4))
 (via (at 131.11481 97.059526) (size 0.889) (drill 0.635) (layers F.Cu B.Cu) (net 4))
 (segment (start 130.9393 75.784) (end 130.9393 96.884016) (width 0.254) (layer F.Cu) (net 4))
 (segment (start 130.9393 75.784) (end 130.9393 76.638) (width 0.254) (layer F.Cu) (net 4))
 (segment (start 131.5893 75.784) (end 131.5893 73.8551) (width 0.254) (layer F.Cu) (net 5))
 (segment (start 131.5893 73.8551) (end 130.7846 73.0504) (width 0.254) (layer F.Cu) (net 5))
 (segment (start 128.383299 78.626701) (end 124.206 82.804) (width 0.254) (layer F.Cu) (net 5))
 (segment (start 130.7846 73.0504) (end 129.2352 73.0504) (width 0.254) (layer F.Cu) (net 5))
 (segment (start 129.2352 73.0504) (end 128.383299 73.902301) (width 0.254) (layer F.Cu) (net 5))
 (segment (start 128.383299 73.902301) (end 128.383299 78.626701) (width 0.254) (layer F.Cu) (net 5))
 (segment (start 131.5893 77.216) (end 131.5893 89.154) (width 0.254) (layer F.Cu) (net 5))
 (segment (start 131.5893 75.784) (end 131.5893 77.216) (width 0.254) (layer F.Cu) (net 5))
 (segment (start 131.5893 77.216) (end 131.5893 77.9953) (width 0.254) (layer F.Cu) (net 5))
 (segment (start 131.5893 77.9953) (end 136.398 82.804) (width 0.254) (layer F.Cu) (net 5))
 (segment (start 131.5893 89.154) (end 131.5893 89.408) (width 0.254) (layer F.Cu) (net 5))
 (segment (start 131.5893 107.2206) (end 131.5893 97.806778) (width 0.254) (layer F.Cu) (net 5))
 (segment (start 131.5893 97.806778) (end 131.940311 97.455767) (width 0.254) (layer F.Cu) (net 5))
 (segment (start 131.940311 97.455767) (end 131.940311 96.663285) (width 0.254) (layer F.Cu) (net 5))
 (segment (start 131.940311 96.663285) (end 131.5893 96.312274) (width 0.254) (layer F.Cu) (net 5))
 (segment (start 131.5893 96.312274) (end 131.5893 89.154) (width 0.254) (layer F.Cu) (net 5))
 (segment (start 131.5893 106.8456) (end 131.5893 107.2206) (width 0.254) (layer F.Cu) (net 5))
 (segment (start 131.5893 89.408) (end 132.0183 89.837) (width 0.254) (layer F.Cu) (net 5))
 (segment (start 133.604 92.898) (end 133.604 91.4227) (width 0.254) (layer F.Cu) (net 5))
 (segment (start 133.604 91.4227) (end 131.5893 89.408) (width 0.254) (layer F.Cu) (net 5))
 (segment (start 131.5893 75.784) (end 131.5893 76.159) (width 0.254) (layer F.Cu) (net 5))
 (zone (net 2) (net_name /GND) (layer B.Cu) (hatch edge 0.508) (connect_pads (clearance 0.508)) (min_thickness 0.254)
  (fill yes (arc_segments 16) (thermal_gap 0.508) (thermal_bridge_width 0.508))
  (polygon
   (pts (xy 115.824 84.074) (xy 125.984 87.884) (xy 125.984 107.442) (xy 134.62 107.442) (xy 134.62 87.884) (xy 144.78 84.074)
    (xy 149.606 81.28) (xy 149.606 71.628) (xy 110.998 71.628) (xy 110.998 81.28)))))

